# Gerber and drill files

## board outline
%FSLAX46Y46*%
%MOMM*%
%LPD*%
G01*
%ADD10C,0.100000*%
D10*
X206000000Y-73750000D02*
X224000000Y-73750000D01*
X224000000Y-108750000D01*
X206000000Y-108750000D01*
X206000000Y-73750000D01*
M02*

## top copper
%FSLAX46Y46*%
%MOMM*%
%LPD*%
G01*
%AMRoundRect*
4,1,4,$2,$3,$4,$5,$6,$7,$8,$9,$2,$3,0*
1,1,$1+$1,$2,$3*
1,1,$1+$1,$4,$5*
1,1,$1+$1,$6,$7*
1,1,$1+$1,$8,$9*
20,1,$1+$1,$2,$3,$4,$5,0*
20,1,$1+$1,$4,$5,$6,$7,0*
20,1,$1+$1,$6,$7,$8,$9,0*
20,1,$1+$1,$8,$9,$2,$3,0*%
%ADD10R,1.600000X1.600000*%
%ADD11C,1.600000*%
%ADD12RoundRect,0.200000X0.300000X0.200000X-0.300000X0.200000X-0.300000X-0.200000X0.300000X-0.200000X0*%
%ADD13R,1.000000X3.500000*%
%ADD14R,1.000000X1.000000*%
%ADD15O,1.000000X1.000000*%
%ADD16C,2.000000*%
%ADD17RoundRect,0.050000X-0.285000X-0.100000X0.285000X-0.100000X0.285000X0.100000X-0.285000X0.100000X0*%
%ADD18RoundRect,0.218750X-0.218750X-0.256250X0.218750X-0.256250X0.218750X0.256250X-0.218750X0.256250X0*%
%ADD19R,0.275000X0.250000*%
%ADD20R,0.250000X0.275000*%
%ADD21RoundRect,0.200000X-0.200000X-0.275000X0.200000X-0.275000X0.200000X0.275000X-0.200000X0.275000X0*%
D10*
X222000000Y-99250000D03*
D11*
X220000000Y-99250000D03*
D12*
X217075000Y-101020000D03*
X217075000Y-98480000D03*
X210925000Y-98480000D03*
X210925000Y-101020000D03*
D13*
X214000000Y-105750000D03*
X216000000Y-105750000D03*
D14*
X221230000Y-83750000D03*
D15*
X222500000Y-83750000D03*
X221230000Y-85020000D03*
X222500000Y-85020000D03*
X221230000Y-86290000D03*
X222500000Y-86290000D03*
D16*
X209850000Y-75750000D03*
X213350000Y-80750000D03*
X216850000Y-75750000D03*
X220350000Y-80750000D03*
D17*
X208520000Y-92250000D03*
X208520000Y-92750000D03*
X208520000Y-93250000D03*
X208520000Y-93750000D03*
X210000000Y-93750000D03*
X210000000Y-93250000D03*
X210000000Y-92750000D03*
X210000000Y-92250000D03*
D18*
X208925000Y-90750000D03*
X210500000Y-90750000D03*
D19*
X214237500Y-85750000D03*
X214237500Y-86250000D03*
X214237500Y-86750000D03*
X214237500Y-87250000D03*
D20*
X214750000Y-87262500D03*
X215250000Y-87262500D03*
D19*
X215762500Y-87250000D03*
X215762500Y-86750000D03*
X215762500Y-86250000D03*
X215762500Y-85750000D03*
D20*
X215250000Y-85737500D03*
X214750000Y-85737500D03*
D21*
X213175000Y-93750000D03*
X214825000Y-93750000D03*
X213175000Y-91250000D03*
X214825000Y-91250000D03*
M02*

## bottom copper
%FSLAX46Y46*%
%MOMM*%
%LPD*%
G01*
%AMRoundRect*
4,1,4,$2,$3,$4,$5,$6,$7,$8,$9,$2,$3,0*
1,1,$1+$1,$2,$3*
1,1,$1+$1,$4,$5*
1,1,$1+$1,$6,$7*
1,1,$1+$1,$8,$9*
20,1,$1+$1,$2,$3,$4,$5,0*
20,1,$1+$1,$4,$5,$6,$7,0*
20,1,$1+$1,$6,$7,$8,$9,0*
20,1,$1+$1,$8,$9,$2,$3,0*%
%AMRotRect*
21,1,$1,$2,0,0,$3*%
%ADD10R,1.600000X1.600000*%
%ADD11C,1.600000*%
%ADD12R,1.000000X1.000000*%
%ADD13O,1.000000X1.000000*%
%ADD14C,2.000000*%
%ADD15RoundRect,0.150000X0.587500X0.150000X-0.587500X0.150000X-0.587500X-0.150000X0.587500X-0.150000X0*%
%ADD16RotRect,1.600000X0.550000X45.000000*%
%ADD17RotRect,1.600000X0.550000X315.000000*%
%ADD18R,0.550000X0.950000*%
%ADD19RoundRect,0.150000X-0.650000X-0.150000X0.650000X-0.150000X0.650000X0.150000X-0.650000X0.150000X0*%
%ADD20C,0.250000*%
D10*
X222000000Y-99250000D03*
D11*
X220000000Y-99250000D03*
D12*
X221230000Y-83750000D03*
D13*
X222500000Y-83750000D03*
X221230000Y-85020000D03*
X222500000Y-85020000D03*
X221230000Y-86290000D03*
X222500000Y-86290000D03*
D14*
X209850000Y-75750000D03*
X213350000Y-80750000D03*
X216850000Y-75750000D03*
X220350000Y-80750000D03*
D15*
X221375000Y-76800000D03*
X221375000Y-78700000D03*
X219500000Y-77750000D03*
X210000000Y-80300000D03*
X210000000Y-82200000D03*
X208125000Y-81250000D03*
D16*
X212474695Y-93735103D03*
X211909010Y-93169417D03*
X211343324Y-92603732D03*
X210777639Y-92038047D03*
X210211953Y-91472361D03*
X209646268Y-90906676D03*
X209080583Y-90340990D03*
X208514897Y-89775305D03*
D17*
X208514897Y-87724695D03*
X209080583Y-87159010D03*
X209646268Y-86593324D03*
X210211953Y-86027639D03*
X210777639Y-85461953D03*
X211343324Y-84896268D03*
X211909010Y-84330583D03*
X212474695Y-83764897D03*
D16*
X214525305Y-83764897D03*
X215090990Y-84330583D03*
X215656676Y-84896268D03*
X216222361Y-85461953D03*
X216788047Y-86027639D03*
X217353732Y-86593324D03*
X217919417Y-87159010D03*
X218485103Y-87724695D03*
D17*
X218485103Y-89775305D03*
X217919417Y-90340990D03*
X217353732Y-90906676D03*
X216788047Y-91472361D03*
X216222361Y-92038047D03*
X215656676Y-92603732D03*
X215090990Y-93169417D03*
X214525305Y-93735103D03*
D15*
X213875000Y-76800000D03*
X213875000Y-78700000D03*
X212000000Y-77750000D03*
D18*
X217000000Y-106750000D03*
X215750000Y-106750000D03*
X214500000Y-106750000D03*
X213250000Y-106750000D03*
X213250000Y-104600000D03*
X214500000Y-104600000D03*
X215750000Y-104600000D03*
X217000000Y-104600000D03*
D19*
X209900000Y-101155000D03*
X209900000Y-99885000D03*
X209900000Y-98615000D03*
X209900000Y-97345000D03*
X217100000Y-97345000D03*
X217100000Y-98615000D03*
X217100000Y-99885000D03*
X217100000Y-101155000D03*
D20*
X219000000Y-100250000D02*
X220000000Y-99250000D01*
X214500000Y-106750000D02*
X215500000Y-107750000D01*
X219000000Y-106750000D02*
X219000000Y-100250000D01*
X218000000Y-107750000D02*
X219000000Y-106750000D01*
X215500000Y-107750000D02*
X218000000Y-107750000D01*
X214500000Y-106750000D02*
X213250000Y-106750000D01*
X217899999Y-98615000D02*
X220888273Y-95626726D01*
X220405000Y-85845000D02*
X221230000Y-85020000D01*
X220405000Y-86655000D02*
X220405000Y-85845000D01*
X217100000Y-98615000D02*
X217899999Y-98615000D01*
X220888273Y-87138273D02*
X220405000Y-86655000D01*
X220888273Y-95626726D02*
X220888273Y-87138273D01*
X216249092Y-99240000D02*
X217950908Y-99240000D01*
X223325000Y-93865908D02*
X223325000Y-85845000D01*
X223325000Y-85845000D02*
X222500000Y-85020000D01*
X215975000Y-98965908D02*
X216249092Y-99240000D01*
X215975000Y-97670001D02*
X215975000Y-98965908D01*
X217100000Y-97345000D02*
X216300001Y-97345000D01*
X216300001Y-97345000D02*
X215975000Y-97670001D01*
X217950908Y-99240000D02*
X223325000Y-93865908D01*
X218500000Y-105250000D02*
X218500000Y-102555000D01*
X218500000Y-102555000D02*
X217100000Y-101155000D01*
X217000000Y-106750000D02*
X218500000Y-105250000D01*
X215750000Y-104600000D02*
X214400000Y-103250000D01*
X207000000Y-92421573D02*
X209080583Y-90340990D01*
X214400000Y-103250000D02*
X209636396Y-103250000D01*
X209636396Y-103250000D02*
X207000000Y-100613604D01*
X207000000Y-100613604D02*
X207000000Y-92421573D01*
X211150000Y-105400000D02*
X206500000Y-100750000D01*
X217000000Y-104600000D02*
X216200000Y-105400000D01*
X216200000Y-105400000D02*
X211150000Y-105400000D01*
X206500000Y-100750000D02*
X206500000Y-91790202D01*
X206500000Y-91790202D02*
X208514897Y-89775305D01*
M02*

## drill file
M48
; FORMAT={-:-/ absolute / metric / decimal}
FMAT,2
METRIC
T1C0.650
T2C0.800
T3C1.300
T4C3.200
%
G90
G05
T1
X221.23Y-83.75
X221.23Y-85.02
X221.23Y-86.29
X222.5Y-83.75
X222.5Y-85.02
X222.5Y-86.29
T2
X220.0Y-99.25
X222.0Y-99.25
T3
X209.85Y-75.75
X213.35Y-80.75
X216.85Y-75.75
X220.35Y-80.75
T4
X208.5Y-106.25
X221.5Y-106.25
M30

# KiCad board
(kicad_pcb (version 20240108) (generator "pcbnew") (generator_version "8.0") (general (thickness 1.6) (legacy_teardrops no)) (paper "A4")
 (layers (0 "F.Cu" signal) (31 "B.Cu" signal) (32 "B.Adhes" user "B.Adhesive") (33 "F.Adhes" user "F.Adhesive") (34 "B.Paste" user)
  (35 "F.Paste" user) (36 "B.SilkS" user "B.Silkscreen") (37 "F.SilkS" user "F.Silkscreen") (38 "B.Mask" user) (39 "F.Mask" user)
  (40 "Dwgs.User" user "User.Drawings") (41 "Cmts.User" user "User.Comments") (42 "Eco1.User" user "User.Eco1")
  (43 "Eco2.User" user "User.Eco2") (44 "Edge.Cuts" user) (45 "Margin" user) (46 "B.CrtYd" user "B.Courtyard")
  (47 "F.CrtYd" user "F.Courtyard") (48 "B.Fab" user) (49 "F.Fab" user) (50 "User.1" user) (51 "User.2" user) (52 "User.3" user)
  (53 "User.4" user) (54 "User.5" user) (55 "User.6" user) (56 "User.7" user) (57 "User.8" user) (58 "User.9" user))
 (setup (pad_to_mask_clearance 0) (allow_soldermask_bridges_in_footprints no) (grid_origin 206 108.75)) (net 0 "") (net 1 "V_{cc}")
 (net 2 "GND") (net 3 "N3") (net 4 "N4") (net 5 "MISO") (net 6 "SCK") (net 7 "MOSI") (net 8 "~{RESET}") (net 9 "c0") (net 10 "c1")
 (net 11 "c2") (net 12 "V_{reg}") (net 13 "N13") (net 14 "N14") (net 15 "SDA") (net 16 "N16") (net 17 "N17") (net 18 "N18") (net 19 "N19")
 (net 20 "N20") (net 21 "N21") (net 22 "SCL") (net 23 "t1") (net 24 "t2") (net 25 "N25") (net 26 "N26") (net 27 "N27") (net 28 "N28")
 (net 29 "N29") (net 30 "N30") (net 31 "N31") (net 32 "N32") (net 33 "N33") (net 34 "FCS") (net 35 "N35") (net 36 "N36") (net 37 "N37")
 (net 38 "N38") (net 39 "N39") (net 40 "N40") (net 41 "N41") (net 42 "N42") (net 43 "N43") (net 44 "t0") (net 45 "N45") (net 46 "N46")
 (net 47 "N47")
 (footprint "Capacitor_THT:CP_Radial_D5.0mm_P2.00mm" (layer "F.Cu") (at 222 99.25 180)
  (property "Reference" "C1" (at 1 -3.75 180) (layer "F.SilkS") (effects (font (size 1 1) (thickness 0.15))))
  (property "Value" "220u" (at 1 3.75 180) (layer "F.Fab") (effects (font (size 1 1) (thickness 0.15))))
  (pad "1" thru_hole rect (at 0 0 180) (size 1.6 1.6) (drill 0.8) (layers "*.Cu" "*.Mask") (remove_unused_layers no) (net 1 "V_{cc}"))
  (pad "2" thru_hole circle (at 2 0 180) (size 1.6 1.6) (drill 0.8) (layers "*.Cu" "*.Mask") (remove_unused_layers no) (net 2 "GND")))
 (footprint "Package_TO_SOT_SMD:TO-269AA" (layer "F.Cu") (at 214 99.75 180)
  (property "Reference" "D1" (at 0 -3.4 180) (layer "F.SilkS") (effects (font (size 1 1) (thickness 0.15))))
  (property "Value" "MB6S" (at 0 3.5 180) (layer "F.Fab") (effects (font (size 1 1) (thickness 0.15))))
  (pad "1" smd roundrect (at -3.075 -1.27 180) (size 1 0.8) (layers "F.Cu" "F.Paste" "F.Mask") (roundrect_rratio 0.25) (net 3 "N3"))
  (pad "2" smd roundrect (at -3.075 1.27 180) (size 1 0.8) (layers "F.Cu" "F.Paste" "F.Mask") (roundrect_rratio 0.25) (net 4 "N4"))
  (pad "3" smd roundrect (at 3.075 1.27 180) (size 1 0.8) (layers "F.Cu" "F.Paste" "F.Mask") (roundrect_rratio 0.25) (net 1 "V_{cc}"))
  (pad "4" smd roundrect (at 3.075 -1.27 180) (size 1 0.8) (layers "F.Cu" "F.Paste" "F.Mask") (roundrect_rratio 0.25) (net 2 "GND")))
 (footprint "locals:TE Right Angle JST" (layer "F.Cu") (at 214 105.75)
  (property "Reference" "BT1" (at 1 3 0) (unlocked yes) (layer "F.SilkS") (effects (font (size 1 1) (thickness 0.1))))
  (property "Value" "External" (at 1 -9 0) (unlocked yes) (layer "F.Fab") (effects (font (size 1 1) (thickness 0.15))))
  (pad "1" smd rect (at 0 0) (size 1 3.5) (layers "F.Cu" "F.Paste" "F.Mask") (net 4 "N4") (thermal_bridge_angle 45))
  (pad "2" smd rect (at 2 0) (size 1 3.5) (layers "F.Cu" "F.Paste" "F.Mask") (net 3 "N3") (thermal_bridge_angle 45)))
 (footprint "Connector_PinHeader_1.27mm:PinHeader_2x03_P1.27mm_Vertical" (layer "F.Cu") (at 221.23 83.75)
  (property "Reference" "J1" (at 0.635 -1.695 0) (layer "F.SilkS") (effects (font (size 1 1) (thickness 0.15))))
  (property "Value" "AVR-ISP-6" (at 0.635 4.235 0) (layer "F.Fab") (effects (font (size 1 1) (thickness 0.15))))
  (pad "1" thru_hole rect (at 0 0) (size 1 1) (drill 0.65) (layers "*.Cu" "*.Mask") (remove_unused_layers no) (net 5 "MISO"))
  (pad "2" thru_hole oval (at 1.27 0) (size 1 1) (drill 0.65) (layers "*.Cu" "*.Mask") (remove_unused_layers no) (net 2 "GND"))
  (pad "3" thru_hole oval (at 0 1.27) (size 1 1) (drill 0.65) (layers "*.Cu" "*.Mask") (remove_unused_layers no) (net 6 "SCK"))
  (pad "4" thru_hole oval (at 1.27 1.27) (size 1 1) (drill 0.65) (layers "*.Cu" "*.Mask") (remove_unused_layers no) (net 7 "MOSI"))
  (pad "5" thru_hole oval (at 0 2.54) (size 1 1) (drill 0.65) (layers "*.Cu" "*.Mask") (remove_unused_layers no) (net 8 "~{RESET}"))
  (pad "6" thru_hole oval (at 1.27 2.54) (size 1 1) (drill 0.65) (layers "*.Cu" "*.Mask") (remove_unused_layers no) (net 1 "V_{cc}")))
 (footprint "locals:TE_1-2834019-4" (layer "F.Cu") (at 207.65 83.45)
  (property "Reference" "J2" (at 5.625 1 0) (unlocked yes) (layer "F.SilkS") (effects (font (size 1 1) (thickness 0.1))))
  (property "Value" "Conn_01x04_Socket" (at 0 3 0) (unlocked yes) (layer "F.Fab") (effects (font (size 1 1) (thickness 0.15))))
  (pad "1" thru_hole circle (at 2.2 -7.7) (size 2 2) (drill 1.3) (layers "*.Cu" "*.Mask") (remove_unused_layers no) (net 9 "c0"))
  (pad "2" thru_hole circle (at 5.7 -2.7) (size 2 2) (drill 1.3) (layers "*.Cu" "*.Mask") (remove_unused_layers no) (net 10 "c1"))
  (pad "3" thru_hole circle (at 9.2 -7.7) (size 2 2) (drill 1.3) (layers "*.Cu" "*.Mask") (remove_unused_layers no) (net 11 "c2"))
  (pad "4" thru_hole circle (at 12.7 -2.7) (size 2 2) (drill 1.3) (layers "*.Cu" "*.Mask") (remove_unused_layers no) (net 2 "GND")))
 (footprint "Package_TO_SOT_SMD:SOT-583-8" (layer "F.Cu") (at 209.26 93)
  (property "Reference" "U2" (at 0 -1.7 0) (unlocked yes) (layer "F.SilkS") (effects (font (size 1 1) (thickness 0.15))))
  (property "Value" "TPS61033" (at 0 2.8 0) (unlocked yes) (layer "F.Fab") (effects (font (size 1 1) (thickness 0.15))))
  (pad "1" smd roundrect (at -0.74 -0.75) (size 0.67 0.3) (layers "F.Cu" "F.Paste" "F.Mask") (roundrect_rratio 0.1666666667)
   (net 1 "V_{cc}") (thermal_bridge_angle 45))
  (pad "2" smd roundrect (at -0.74 -0.25) (size 0.67 0.3) (layers "F.Cu" "F.Paste" "F.Mask") (roundrect_rratio 0.1666666667)
   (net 1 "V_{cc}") (thermal_bridge_angle 45))
  (pad "3" smd roundrect (at -0.74 0.25) (size 0.67 0.3) (layers "F.Cu" "F.Paste" "F.Mask") (roundrect_rratio 0.1666666667) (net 1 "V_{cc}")
   (thermal_bridge_angle 45))
  (pad "4" smd roundrect (at -0.74 0.75) (size 0.67 0.3) (layers "F.Cu" "F.Paste" "F.Mask") (roundrect_rratio 0.1666666667)
   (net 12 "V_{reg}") (thermal_bridge_angle 45))
  (pad "5" smd roundrect (at 0.74 0.75) (size 0.67 0.3) (layers "F.Cu" "F.Paste" "F.Mask") (roundrect_rratio 0.1666666667) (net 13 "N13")
   (thermal_bridge_angle 45))
  (pad "6" smd roundrect (at 0.74 0.25) (size 0.67 0.3) (layers "F.Cu" "F.Paste" "F.Mask") (roundrect_rratio 0.1666666667) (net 2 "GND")
   (thermal_bridge_angle 45))
  (pad "7" smd roundrect (at 0.74 -0.25) (size 0.67 0.3) (layers "F.Cu" "F.Paste" "F.Mask") (roundrect_rratio 0.1666666667) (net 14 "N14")
   (thermal_bridge_angle 45))
  (pad "8" smd roundrect (at 0.74 -0.75) (size 0.67 0.3) (layers "F.Cu" "F.Paste" "F.Mask") (roundrect_rratio 0.1666666667)
   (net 12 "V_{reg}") (thermal_bridge_angle 45)))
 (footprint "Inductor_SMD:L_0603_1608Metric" (layer "F.Cu") (at 209.7125 90.75)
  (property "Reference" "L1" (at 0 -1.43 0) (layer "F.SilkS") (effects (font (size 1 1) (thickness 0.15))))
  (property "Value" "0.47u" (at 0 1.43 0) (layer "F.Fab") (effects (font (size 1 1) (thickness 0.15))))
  (pad "1" smd roundrect (at -0.7875 0) (size 0.875 0.95) (layers "F.Cu" "F.Paste" "F.Mask") (roundrect_rratio 0.25) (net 14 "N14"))
  (pad "2" smd roundrect (at 0.7875 0) (size 0.875 0.95) (layers "F.Cu" "F.Paste" "F.Mask") (roundrect_rratio 0.25) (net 1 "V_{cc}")))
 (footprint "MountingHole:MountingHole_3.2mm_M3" (layer "F.Cu") (at 208.5 106.25)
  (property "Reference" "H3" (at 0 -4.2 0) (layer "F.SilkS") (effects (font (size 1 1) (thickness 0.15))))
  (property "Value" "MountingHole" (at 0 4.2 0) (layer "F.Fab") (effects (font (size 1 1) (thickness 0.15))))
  (pad "" np_thru_hole circle (at 0 0) (size 3.2 3.2) (drill 3.2) (layers "*.Cu" "*.Mask")))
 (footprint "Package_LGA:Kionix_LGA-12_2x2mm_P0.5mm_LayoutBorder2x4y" (layer "F.Cu") (at 215 86.5)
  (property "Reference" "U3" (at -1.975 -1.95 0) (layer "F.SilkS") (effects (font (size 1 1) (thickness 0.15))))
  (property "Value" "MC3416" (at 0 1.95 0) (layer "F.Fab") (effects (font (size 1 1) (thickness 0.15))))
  (pad "1" smd rect (at -0.7625 -0.75) (size 0.275 0.25) (layers "F.Cu" "F.Paste" "F.Mask") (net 2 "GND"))
  (pad "2" smd rect (at -0.7625 -0.25) (size 0.275 0.25) (layers "F.Cu" "F.Paste" "F.Mask") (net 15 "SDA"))
  (pad "3" smd rect (at -0.7625 0.25) (size 0.275 0.25) (layers "F.Cu" "F.Paste" "F.Mask") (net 12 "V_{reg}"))
  (pad "4" smd rect (at -0.7625 0.75) (size 0.275 0.25) (layers "F.Cu" "F.Paste" "F.Mask") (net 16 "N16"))
  (pad "5" smd rect (at -0.25 0.7625) (size 0.25 0.275) (layers "F.Cu" "F.Paste" "F.Mask") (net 12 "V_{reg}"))
  (pad "6" smd rect (at 0.25 0.7625) (size 0.25 0.275) (layers "F.Cu" "F.Paste" "F.Mask") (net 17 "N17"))
  (pad "7" smd rect (at 0.7625 0.75) (size 0.275 0.25) (layers "F.Cu" "F.Paste" "F.Mask") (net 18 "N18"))
  (pad "8" smd rect (at 0.7625 0.25) (size 0.275 0.25) (layers "F.Cu" "F.Paste" "F.Mask") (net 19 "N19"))
  (pad "9" smd rect (at 0.7625 -0.25) (size 0.275 0.25) (layers "F.Cu" "F.Paste" "F.Mask") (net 2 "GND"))
  (pad "10" smd rect (at 0.7625 -0.75) (size 0.275 0.25) (layers "F.Cu" "F.Paste" "F.Mask") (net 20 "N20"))
  (pad "11" smd rect (at 0.25 -0.7625) (size 0.25 0.275) (layers "F.Cu" "F.Paste" "F.Mask") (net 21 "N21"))
  (pad "12" smd rect (at -0.25 -0.7625) (size 0.25 0.275) (layers "F.Cu" "F.Paste" "F.Mask") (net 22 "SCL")))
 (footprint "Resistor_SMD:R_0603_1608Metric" (layer "F.Cu") (at 214 93.75)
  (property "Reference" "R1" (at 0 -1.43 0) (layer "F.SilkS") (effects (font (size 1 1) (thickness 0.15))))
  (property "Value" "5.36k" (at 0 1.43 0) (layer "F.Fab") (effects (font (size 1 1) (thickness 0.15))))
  (pad "1" smd roundrect (at -0.825 0) (size 0.8 0.95) (layers "F.Cu" "F.Paste" "F.Mask") (roundrect_rratio 0.25) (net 12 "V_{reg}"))
  (pad "2" smd roundrect (at 0.825 0) (size 0.8 0.95) (layers "F.Cu" "F.Paste" "F.Mask") (roundrect_rratio 0.25) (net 13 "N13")))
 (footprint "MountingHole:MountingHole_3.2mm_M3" (layer "F.Cu") (at 221.5 106.25)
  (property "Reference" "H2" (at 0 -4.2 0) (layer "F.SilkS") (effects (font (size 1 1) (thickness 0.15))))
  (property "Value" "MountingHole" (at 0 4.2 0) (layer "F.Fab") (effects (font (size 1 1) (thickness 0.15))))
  (pad "" np_thru_hole circle (at 0 0) (size 3.2 3.2) (drill 3.2) (layers "*.Cu" "*.Mask")))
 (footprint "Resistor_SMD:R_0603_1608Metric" (layer "F.Cu") (at 214 91.25)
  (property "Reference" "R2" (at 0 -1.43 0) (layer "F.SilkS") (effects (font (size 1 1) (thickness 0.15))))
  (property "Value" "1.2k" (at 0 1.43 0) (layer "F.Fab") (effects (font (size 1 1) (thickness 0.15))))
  (pad "1" smd roundrect (at -0.825 0) (size 0.8 0.95) (layers "F.Cu" "F.Paste" "F.Mask") (roundrect_rratio 0.25) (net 13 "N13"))
  (pad "2" smd roundrect (at 0.825 0) (size 0.8 0.95) (layers "F.Cu" "F.Paste" "F.Mask") (roundrect_rratio 0.25) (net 2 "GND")))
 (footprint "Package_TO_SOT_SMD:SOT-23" (layer "B.Cu") (at 220.4375 77.75 180)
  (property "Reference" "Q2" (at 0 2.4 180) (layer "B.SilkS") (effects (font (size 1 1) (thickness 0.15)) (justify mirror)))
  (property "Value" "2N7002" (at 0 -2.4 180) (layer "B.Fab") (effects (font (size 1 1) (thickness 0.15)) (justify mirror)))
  (pad "1" smd roundrect (at -0.9375 0.95 180) (size 1.475 0.6) (layers "B.Cu" "B.Paste" "B.Mask") (roundrect_rratio 0.25) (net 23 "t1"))
  (pad "2" smd roundrect (at -0.9375 -0.95 180) (size 1.475 0.6) (layers "B.Cu" "B.Paste" "B.Mask") (roundrect_rratio 0.25) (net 10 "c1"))
  (pad "3" smd roundrect (at 0.9375 0 180) (size 1.475 0.6) (layers "B.Cu" "B.Paste" "B.Mask") (roundrect_rratio 0.25) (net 1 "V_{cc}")))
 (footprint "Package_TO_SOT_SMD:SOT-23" (layer "B.Cu") (at 209.0625 81.25 180)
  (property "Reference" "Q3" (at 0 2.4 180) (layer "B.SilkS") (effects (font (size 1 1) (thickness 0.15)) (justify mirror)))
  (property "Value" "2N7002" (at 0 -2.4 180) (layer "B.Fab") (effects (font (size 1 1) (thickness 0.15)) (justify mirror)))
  (pad "1" smd roundrect (at -0.9375 0.95 180) (size 1.475 0.6) (layers "B.Cu" "B.Paste" "B.Mask") (roundrect_rratio 0.25) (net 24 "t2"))
  (pad "2" smd roundrect (at -0.9375 -0.95 180) (size 1.475 0.6) (layers "B.Cu" "B.Paste" "B.Mask") (roundrect_rratio 0.25) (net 11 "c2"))
  (pad "3" smd roundrect (at 0.9375 0 180) (size 1.475 0.6) (layers "B.Cu" "B.Paste" "B.Mask") (roundrect_rratio 0.25) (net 1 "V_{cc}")))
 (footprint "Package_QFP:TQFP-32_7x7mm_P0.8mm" (layer "B.Cu") (at 213.5 88.75 45)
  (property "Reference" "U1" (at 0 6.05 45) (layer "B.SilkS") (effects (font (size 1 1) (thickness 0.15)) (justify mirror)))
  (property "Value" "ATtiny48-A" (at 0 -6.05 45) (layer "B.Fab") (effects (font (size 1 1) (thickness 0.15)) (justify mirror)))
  (pad "1" smd rect (at -4.25 2.8 45) (size 1.6 0.55) (layers "B.Cu" "B.Paste" "B.Mask") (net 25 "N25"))
  (pad "2" smd rect (at -4.25 2 45) (size 1.6 0.55) (layers "B.Cu" "B.Paste" "B.Mask") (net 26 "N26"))
  (pad "3" smd rect (at -4.25 1.2 45) (size 1.6 0.55) (layers "B.Cu" "B.Paste" "B.Mask") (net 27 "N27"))
  (pad "4" smd rect (at -4.25 0.4 45) (size 1.6 0.55) (layers "B.Cu" "B.Paste" "B.Mask") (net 12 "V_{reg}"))
  (pad "5" smd rect (at -4.25 -0.4 45) (size 1.6 0.55) (layers "B.Cu" "B.Paste" "B.Mask") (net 2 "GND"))
  (pad "6" smd rect (at -4.25 -1.2 45) (size 1.6 0.55) (layers "B.Cu" "B.Paste" "B.Mask") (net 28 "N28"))
  (pad "7" smd rect (at -4.25 -2 45) (size 1.6 0.55) (layers "B.Cu" "B.Paste" "B.Mask") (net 15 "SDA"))
  (pad "8" smd rect (at -4.25 -2.8 45) (size 1.6 0.55) (layers "B.Cu" "B.Paste" "B.Mask") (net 22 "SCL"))
  (pad "9" smd rect (at -2.8 -4.25 315) (size 1.6 0.55) (layers "B.Cu" "B.Paste" "B.Mask") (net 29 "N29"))
  (pad "10" smd rect (at -2 -4.25 315) (size 1.6 0.55) (layers "B.Cu" "B.Paste" "B.Mask") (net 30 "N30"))
  (pad "11" smd rect (at -1.2 -4.25 315) (size 1.6 0.55) (layers "B.Cu" "B.Paste" "B.Mask") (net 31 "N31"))
  (pad "12" smd rect (at -0.4 -4.25 315) (size 1.6 0.55) (layers "B.Cu" "B.Paste" "B.Mask") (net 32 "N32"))
  (pad "13" smd rect (at 0.4 -4.25 315) (size 1.6 0.55) (layers "B.Cu" "B.Paste" "B.Mask") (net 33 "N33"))
  (pad "14" smd rect (at 1.2 -4.25 315) (size 1.6 0.55) (layers "B.Cu" "B.Paste" "B.Mask") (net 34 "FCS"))
  (pad "15" smd rect (at 2 -4.25 315) (size 1.6 0.55) (layers "B.Cu" "B.Paste" "B.Mask") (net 7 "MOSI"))
  (pad "16" smd rect (at 2.8 -4.25 315) (size 1.6 0.55) (layers "B.Cu" "B.Paste" "B.Mask") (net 5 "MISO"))
  (pad "17" smd rect (at 4.25 -2.8 45) (size 1.6 0.55) (layers "B.Cu" "B.Paste" "B.Mask") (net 6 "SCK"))
  (pad "18" smd rect (at 4.25 -2 45) (size 1.6 0.55) (layers "B.Cu" "B.Paste" "B.Mask") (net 12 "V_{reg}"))
  (pad "19" smd rect (at 4.25 -1.2 45) (size 1.6 0.55) (layers "B.Cu" "B.Paste" "B.Mask") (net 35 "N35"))
  (pad "20" smd rect (at 4.25 -0.4 45) (size 1.6 0.55) (layers "B.Cu" "B.Paste" "B.Mask") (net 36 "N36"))
  (pad "21" smd rect (at 4.25 0.4 45) (size 1.6 0.55) (layers "B.Cu" "B.Paste" "B.Mask") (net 2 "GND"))
  (pad "22" smd rect (at 4.25 1.2 45) (size 1.6 0.55) (layers "B.Cu" "B.Paste" "B.Mask") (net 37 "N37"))
  (pad "23" smd rect (at 4.25 2 45) (size 1.6 0.55) (layers "B.Cu" "B.Paste" "B.Mask") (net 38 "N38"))
  (pad "24" smd rect (at 4.25 2.8 45) (size 1.6 0.55) (layers "B.Cu" "B.Paste" "B.Mask") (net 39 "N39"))
  (pad "25" smd rect (at 2.8 4.25 315) (size 1.6 0.55) (layers "B.Cu" "B.Paste" "B.Mask") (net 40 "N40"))
  (pad "26" smd rect (at 2 4.25 315) (size 1.6 0.55) (layers "B.Cu" "B.Paste" "B.Mask") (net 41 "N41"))
  (pad "27" smd rect (at 1.2 4.25 315) (size 1.6 0.55) (layers "B.Cu" "B.Paste" "B.Mask") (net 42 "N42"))
  (pad "28" smd rect (at 0.4 4.25 315) (size 1.6 0.55) (layers "B.Cu" "B.Paste" "B.Mask") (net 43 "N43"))
  (pad "29" smd rect (at -0.4 4.25 315) (size 1.6 0.55) (layers "B.Cu" "B.Paste" "B.Mask") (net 8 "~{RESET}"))
  (pad "30" smd rect (at -1.2 4.25 315) (size 1.6 0.55) (layers "B.Cu" "B.Paste" "B.Mask") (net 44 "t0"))
  (pad "31" smd rect (at -2 4.25 315) (size 1.6 0.55) (layers "B.Cu" "B.Paste" "B.Mask") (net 23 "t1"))
  (pad "32" smd rect (at -2.8 4.25 315) (size 1.6 0.55) (layers "B.Cu" "B.Paste" "B.Mask") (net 24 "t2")))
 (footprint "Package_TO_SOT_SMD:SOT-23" (layer "B.Cu") (at 212.9375 77.75 180)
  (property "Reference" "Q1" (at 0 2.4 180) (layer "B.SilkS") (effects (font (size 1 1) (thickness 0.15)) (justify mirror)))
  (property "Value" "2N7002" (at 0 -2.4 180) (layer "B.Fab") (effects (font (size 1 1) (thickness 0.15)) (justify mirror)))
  (pad "1" smd roundrect (at -0.9375 0.95 180) (size 1.475 0.6) (layers "B.Cu" "B.Paste" "B.Mask") (roundrect_rratio 0.25) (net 44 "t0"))
  (pad "2" smd roundrect (at -0.9375 -0.95 180) (size 1.475 0.6) (layers "B.Cu" "B.Paste" "B.Mask") (roundrect_rratio 0.25) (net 9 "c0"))
  (pad "3" smd roundrect (at 0.9375 0 180) (size 1.475 0.6) (layers "B.Cu" "B.Paste" "B.Mask") (roundrect_rratio 0.25) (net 1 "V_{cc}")))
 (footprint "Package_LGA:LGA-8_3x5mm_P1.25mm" (layer "B.Cu") (at 215.125 105.675 90)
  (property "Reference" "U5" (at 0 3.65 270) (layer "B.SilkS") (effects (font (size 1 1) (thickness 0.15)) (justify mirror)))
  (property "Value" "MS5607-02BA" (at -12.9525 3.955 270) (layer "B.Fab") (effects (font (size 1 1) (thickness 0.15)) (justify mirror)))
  (pad "1" smd rect (at -1.075 1.875 90) (size 0.95 0.55) (layers "B.Cu" "B.Paste" "B.Mask") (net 12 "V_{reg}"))
  (pad "2" smd rect (at -1.075 0.625 90) (size 0.95 0.55) (layers "B.Cu" "B.Paste" "B.Mask") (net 12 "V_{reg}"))
  (pad "3" smd rect (at -1.075 -0.625 90) (size 0.95 0.55) (layers "B.Cu" "B.Paste" "B.Mask") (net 2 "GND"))
  (pad "4" smd rect (at -1.075 -1.875 90) (size 0.95 0.55) (layers "B.Cu" "B.Paste" "B.Mask") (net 2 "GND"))
  (pad "5" smd rect (at 1.075 -1.875 90) (size 0.95 0.55) (layers "B.Cu" "B.Paste" "B.Mask") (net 2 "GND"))
  (pad "6" smd rect (at 1.075 -0.625 90) (size 0.95 0.55) (layers "B.Cu" "B.Paste" "B.Mask") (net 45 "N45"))
  (pad "7" smd rect (at 1.075 0.625 90) (size 0.95 0.55) (layers "B.Cu" "B.Paste" "B.Mask") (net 15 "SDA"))
  (pad "8" smd rect (at 1.075 1.875 90) (size 0.95 0.55) (layers "B.Cu" "B.Paste" "B.Mask") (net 22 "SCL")))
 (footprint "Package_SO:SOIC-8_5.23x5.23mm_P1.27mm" (layer "B.Cu") (at 213.5 99.25)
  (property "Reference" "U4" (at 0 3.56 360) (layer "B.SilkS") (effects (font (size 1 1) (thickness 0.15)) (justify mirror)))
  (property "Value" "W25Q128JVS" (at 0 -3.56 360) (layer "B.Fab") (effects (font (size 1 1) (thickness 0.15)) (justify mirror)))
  (pad "1" smd roundrect (at -3.6 1.905) (size 1.6 0.6) (layers "B.Cu" "B.Paste" "B.Mask") (roundrect_rratio 0.25) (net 34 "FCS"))
  (pad "2" smd roundrect (at -3.6 0.635) (size 1.6 0.6) (layers "B.Cu" "B.Paste" "B.Mask") (roundrect_rratio 0.25) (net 5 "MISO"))
  (pad "3" smd roundrect (at -3.6 -0.635) (size 1.6 0.6) (layers "B.Cu" "B.Paste" "B.Mask") (roundrect_rratio 0.25) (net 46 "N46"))
  (pad "4" smd roundrect (at -3.6 -1.905) (size 1.6 0.6) (layers "B.Cu" "B.Paste" "B.Mask") (roundrect_rratio 0.25) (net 2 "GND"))
  (pad "5" smd roundrect (at 3.6 -1.905) (size 1.6 0.6) (layers "B.Cu" "B.Paste" "B.Mask") (roundrect_rratio 0.25) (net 7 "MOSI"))
  (pad "6" smd roundrect (at 3.6 -0.635) (size 1.6 0.6) (layers "B.Cu" "B.Paste" "B.Mask") (roundrect_rratio 0.25) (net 6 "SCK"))
  (pad "7" smd roundrect (at 3.6 0.635) (size 1.6 0.6) (layers "B.Cu" "B.Paste" "B.Mask") (roundrect_rratio 0.25) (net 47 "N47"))
  (pad "8" smd roundrect (at 3.6 1.905) (size 1.6 0.6) (layers "B.Cu" "B.Paste" "B.Mask") (roundrect_rratio 0.25) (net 12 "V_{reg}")))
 (gr_rect (start 206 73.75) (end 224 108.75) (stroke (width 0.1) (type default)) (fill none) (layer "Edge.Cuts"))
 (segment (start 219 100.25) (end 220 99.25) (width 0.25) (layer "B.Cu") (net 2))
 (segment (start 214.5 106.75) (end 215.5 107.75) (width 0.25) (layer "B.Cu") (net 2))
 (segment (start 219 106.75) (end 219 100.25) (width 0.25) (layer "B.Cu") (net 2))
 (segment (start 218 107.75) (end 219 106.75) (width 0.25) (layer "B.Cu") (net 2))
 (segment (start 215.5 107.75) (end 218 107.75) (width 0.25) (layer "B.Cu") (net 2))
 (segment (start 214.5 106.75) (end 213.25 106.75) (width 0.25) (layer "B.Cu") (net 2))
 (segment (start 217.899999 98.615) (end 220.888273 95.626726) (width 0.25) (layer "B.Cu") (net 6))
 (segment (start 220.405 85.845) (end 221.23 85.02) (width 0.25) (layer "B.Cu") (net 6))
 (segment (start 220.405 86.655) (end 220.405 85.845) (width 0.25) (layer "B.Cu") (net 6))
 (segment (start 217.1 98.615) (end 217.899999 98.615) (width 0.25) (layer "B.Cu") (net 6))
 (segment (start 220.888273 87.138273) (end 220.405 86.655) (width 0.25) (layer "B.Cu") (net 6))
 (segment (start 220.888273 95.626726) (end 220.888273 87.138273) (width 0.25) (layer "B.Cu") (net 6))
 (segment (start 216.249092 99.24) (end 217.950908 99.24) (width 0.25) (layer "B.Cu") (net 7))
 (segment (start 223.325 93.865908) (end 223.325 85.845) (width 0.25) (layer "B.Cu") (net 7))
 (segment (start 223.325 85.845) (end 222.5 85.02) (width 0.25) (layer "B.Cu") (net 7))
 (segment (start 215.975 98.965908) (end 216.249092 99.24) (width 0.25) (layer "B.Cu") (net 7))
 (segment (start 215.975 97.670001) (end 215.975 98.965908) (width 0.25) (layer "B.Cu") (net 7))
 (segment (start 217.1 97.345) (end 216.300001 97.345) (width 0.25) (layer "B.Cu") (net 7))
 (segment (start 216.300001 97.345) (end 215.975 97.670001) (width 0.25) (layer "B.Cu") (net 7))
 (segment (start 217.950908 99.24) (end 223.325 93.865908) (width 0.25) (layer "B.Cu") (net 7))
 (segment (start 218.5 105.25) (end 218.5 102.555) (width 0.25) (layer "B.Cu") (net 12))
 (segment (start 218.5 102.555) (end 217.1 101.155) (width 0.25) (layer "B.Cu") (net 12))
 (segment (start 217 106.75) (end 218.5 105.25) (width 0.25) (layer "B.Cu") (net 12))
 (segment (start 215.75 104.6) (end 214.4 103.25) (width 0.25) (layer "B.Cu") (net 15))
 (segment (start 207 92.421573) (end 209.080583 90.34099) (width 0.25) (layer "B.Cu") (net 15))
 (segment (start 214.4 103.25) (end 209.636396 103.25) (width 0.25) (layer "B.Cu") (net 15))
 (segment (start 209.636396 103.25) (end 207 100.613604) (width 0.25) (layer "B.Cu") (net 15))
 (segment (start 207 100.613604) (end 207 92.421573) (width 0.25) (layer "B.Cu") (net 15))
 (segment (start 211.15 105.4) (end 206.5 100.75) (width 0.25) (layer "B.Cu") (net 22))
 (segment (start 217 104.6) (end 216.2 105.4) (width 0.25) (layer "B.Cu") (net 22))
 (segment (start 216.2 105.4) (end 211.15 105.4) (width 0.25) (layer "B.Cu") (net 22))
 (segment (start 206.5 100.75) (end 206.5 91.790202) (width 0.25) (layer "B.Cu") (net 22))
 (segment (start 206.5 91.790202) (end 208.514897 89.775305) (width 0.25) (layer "B.Cu") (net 22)))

